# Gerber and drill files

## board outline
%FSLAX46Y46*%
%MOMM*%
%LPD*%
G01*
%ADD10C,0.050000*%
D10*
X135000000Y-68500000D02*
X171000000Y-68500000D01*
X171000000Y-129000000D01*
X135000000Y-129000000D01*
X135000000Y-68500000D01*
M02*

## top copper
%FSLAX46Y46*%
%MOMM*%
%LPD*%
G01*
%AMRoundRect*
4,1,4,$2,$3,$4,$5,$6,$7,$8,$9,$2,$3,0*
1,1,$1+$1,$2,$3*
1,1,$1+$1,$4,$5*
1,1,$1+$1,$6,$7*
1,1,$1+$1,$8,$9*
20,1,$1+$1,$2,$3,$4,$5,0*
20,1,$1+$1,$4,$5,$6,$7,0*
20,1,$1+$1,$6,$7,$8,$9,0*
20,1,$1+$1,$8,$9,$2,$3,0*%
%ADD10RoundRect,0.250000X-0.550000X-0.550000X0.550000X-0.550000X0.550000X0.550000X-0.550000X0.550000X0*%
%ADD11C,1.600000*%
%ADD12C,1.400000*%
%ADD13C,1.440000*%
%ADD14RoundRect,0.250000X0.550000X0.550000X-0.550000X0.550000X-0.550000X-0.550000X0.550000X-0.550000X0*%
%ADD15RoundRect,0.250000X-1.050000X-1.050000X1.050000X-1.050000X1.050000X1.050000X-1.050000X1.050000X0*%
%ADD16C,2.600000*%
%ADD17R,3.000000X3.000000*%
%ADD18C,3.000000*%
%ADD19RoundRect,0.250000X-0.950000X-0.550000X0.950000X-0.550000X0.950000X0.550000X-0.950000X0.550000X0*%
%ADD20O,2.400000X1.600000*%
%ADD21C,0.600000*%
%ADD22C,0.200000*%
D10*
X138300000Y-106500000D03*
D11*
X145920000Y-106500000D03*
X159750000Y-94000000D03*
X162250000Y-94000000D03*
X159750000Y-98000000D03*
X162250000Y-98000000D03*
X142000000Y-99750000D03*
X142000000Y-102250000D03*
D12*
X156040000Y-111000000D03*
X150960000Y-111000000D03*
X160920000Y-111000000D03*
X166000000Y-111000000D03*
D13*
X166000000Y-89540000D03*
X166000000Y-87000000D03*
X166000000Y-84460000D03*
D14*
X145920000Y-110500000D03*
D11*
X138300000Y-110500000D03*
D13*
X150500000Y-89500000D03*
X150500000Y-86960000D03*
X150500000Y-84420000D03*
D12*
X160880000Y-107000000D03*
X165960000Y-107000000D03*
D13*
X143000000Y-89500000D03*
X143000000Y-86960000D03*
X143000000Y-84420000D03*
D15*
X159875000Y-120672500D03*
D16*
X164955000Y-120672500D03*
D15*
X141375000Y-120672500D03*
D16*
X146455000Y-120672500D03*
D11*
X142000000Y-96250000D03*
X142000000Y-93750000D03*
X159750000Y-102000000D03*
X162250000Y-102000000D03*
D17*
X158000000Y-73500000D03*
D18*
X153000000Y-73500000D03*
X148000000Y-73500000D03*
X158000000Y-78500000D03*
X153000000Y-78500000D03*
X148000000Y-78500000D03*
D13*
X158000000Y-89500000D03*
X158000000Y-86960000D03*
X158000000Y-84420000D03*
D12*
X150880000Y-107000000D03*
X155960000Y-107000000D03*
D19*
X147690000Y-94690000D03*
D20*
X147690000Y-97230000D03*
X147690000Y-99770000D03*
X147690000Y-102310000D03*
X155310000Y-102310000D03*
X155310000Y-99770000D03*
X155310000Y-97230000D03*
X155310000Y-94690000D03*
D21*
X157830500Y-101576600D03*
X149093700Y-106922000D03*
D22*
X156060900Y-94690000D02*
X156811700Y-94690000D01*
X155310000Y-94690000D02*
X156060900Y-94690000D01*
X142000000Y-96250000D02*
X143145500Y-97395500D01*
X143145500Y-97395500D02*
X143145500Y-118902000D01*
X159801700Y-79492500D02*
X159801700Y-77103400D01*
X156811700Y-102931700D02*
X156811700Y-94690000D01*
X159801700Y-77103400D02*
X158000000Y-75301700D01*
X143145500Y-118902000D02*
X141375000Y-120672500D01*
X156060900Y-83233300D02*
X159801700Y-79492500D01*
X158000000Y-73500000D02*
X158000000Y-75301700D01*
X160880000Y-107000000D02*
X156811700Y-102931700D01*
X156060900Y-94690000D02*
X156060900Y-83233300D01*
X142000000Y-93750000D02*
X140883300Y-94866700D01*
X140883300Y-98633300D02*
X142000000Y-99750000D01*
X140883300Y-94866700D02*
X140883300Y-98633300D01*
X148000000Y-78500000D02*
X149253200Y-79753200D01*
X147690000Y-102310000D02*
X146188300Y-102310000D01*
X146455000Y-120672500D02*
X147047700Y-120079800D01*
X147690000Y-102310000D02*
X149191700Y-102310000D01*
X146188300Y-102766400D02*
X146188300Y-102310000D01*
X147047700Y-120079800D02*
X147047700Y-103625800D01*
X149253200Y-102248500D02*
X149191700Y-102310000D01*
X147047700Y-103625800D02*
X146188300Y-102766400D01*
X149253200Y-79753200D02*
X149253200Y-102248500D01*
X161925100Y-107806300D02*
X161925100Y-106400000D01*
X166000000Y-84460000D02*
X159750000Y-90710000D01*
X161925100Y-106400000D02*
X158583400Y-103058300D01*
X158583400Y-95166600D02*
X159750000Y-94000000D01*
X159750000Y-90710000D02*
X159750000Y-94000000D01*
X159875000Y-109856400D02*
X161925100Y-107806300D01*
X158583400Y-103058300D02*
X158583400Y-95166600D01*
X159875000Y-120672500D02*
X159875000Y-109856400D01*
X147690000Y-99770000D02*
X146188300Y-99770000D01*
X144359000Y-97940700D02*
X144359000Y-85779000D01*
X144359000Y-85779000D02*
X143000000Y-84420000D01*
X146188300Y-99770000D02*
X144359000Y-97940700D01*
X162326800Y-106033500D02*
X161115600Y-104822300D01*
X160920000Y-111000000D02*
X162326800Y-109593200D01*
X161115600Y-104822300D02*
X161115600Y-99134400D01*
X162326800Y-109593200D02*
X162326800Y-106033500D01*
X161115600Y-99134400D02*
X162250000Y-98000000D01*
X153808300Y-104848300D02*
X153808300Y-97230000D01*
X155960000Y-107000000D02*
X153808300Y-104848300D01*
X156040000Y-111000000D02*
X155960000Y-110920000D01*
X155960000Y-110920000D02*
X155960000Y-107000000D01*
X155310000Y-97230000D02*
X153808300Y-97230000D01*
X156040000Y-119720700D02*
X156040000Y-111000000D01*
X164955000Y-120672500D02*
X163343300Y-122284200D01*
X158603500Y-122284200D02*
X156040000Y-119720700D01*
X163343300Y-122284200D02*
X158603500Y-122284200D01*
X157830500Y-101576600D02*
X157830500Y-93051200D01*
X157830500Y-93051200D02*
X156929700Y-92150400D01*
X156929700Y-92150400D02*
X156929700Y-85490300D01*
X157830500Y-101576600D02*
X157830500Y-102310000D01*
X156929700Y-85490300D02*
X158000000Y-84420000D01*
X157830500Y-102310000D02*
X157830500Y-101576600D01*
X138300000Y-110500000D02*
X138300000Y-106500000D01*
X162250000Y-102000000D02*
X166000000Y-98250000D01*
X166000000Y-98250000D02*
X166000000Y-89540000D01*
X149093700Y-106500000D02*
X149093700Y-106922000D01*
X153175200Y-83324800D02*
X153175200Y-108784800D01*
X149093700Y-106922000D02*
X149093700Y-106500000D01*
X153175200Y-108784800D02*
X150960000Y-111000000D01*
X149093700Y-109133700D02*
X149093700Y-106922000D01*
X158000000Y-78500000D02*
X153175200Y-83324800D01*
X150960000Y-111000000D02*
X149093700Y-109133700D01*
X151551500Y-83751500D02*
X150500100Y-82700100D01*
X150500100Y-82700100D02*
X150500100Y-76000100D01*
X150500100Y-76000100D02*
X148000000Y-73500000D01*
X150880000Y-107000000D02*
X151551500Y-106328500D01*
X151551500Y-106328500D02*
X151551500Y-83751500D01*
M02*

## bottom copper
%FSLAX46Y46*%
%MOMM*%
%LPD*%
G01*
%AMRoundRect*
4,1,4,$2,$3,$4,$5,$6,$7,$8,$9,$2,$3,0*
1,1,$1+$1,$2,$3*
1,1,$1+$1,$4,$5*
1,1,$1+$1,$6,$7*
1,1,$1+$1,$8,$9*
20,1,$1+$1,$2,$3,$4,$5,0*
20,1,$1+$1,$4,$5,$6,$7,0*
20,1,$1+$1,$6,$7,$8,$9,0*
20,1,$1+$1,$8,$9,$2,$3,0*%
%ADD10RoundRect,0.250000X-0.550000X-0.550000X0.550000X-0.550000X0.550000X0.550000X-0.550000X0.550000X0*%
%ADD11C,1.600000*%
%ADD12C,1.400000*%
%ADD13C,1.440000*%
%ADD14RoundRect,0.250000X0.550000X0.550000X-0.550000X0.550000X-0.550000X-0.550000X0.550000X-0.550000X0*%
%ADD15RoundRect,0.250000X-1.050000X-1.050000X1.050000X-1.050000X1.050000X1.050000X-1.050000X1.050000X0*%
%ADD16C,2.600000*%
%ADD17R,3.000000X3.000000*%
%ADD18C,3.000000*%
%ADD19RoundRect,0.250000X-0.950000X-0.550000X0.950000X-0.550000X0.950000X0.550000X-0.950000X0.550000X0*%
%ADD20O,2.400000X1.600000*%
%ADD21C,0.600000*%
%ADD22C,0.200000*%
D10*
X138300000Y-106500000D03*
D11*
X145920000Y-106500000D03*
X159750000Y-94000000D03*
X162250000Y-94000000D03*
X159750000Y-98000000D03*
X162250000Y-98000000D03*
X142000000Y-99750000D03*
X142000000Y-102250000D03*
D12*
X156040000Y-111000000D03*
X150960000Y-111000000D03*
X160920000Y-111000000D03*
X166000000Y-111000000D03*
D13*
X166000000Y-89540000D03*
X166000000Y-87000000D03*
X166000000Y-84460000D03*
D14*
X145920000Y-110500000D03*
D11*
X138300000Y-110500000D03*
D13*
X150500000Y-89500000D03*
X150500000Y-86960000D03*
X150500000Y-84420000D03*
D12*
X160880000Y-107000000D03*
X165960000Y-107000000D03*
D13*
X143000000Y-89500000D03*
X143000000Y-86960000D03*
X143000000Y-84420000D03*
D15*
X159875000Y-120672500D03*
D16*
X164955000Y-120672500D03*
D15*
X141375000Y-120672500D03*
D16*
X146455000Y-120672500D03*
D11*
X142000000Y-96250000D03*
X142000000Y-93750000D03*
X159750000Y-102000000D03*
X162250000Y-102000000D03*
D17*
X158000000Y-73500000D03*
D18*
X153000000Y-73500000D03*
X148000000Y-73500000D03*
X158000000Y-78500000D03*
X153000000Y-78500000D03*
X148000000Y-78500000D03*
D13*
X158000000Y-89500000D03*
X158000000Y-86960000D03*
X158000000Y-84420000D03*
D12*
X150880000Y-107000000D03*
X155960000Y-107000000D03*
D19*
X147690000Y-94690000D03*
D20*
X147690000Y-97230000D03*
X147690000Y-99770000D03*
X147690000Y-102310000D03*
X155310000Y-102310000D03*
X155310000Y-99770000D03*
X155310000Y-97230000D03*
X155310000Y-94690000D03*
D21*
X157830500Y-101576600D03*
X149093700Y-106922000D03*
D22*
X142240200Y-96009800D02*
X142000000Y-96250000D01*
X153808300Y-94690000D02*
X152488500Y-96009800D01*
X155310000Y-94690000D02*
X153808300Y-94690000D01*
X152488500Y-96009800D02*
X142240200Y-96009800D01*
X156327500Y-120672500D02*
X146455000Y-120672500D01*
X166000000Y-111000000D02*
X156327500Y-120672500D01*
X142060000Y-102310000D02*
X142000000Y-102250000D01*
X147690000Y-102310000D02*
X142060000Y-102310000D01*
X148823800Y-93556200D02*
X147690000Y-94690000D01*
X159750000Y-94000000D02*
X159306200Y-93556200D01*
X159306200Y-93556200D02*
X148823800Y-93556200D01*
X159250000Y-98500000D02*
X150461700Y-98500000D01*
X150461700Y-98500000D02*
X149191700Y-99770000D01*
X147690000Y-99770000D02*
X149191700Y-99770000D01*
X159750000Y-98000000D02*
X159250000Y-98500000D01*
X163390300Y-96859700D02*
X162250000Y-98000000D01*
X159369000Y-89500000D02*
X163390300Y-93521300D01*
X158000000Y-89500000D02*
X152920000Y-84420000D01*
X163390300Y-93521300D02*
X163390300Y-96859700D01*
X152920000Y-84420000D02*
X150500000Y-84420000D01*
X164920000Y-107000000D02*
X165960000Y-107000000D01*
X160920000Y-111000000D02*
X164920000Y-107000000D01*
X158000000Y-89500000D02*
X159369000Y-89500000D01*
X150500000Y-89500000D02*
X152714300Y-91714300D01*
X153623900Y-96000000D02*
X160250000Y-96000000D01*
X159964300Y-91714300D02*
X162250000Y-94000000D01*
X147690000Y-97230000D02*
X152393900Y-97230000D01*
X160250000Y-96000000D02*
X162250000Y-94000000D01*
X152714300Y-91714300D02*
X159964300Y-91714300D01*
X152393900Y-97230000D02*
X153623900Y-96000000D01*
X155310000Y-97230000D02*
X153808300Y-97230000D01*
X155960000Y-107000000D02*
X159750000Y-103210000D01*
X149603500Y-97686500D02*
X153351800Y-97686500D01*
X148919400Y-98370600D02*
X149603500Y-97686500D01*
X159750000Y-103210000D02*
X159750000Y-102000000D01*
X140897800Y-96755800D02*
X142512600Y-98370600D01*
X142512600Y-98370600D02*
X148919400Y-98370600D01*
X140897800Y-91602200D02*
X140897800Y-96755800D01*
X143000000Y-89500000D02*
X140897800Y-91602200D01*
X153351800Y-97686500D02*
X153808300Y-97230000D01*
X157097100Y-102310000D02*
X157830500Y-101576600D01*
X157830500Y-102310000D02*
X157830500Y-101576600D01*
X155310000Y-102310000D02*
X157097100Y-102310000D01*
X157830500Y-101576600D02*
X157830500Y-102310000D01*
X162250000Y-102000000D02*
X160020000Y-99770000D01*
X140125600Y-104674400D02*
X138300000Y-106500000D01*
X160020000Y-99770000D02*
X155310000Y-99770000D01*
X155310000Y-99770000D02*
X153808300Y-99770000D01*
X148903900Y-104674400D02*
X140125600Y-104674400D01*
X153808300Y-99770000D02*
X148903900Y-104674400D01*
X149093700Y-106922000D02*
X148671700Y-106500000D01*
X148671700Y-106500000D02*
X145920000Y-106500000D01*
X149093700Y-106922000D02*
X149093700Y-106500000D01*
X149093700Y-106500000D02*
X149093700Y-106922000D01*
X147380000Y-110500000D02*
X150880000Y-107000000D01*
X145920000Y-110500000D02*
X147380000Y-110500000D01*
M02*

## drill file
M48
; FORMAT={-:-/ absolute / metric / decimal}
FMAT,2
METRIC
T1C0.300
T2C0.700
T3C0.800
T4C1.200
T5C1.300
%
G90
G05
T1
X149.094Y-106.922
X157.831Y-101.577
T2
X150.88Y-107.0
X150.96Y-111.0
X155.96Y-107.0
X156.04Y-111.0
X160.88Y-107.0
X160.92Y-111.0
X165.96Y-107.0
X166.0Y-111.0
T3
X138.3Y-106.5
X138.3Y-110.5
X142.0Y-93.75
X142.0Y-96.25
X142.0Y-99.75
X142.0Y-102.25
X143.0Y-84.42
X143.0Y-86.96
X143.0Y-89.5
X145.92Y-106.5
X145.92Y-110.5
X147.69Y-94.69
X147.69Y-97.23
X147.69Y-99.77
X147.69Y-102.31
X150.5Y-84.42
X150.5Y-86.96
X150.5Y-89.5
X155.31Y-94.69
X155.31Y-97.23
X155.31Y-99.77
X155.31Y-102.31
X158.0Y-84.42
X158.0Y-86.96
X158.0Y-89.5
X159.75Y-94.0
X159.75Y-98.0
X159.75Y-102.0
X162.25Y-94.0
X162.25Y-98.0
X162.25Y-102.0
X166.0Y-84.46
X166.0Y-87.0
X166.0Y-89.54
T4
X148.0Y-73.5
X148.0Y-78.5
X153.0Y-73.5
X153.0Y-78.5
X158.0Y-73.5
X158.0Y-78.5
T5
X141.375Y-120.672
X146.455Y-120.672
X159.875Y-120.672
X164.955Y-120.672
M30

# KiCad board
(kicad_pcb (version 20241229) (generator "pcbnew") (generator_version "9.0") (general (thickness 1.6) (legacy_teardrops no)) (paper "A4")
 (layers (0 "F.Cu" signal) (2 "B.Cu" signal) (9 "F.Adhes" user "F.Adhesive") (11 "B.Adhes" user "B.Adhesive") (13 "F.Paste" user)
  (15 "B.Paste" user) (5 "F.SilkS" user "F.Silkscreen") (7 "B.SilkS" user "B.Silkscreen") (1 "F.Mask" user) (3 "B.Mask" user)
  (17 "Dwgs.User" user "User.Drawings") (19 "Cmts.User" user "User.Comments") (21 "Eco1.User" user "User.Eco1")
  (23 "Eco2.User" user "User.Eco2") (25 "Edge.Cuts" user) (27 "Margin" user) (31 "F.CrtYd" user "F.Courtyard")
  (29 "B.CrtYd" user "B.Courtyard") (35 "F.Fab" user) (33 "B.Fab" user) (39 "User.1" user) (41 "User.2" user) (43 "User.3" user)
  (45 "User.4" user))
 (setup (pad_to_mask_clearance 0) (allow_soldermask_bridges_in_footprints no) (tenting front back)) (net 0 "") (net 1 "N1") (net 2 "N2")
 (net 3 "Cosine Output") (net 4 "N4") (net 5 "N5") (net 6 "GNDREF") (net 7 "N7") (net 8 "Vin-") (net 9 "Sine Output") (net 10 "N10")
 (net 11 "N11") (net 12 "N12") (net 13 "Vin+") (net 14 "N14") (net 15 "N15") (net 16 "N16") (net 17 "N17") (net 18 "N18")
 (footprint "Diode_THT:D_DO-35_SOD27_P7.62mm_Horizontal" (layer "F.Cu") (at 138.3 106.5)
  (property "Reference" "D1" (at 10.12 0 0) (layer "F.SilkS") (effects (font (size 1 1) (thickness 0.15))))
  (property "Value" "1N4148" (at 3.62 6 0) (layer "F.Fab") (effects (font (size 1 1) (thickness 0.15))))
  (pad "1" thru_hole roundrect (at 0 0) (size 1.6 1.6) (drill 0.8) (layers "*.Cu" "*.Mask") (remove_unused_layers no)
   (roundrect_rratio 0.15625) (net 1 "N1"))
  (pad "2" thru_hole circle (at 7.62 0) (size 1.6 1.6) (drill 0.8) (layers "*.Cu" "*.Mask") (remove_unused_layers no) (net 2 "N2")))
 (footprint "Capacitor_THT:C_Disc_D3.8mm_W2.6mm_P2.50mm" (layer "F.Cu") (at 159.75 94)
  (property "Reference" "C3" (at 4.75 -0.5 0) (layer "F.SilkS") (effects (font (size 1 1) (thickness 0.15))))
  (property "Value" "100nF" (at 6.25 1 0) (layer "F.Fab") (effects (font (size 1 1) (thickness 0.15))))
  (pad "1" thru_hole circle (at 0 0) (size 1.6 1.6) (drill 0.8) (layers "*.Cu" "*.Mask") (remove_unused_layers no) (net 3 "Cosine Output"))
  (pad "2" thru_hole circle (at 2.5 0) (size 1.6 1.6) (drill 0.8) (layers "*.Cu" "*.Mask") (remove_unused_layers no) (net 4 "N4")))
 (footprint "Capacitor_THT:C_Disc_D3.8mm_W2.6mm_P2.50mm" (layer "F.Cu") (at 159.75 98)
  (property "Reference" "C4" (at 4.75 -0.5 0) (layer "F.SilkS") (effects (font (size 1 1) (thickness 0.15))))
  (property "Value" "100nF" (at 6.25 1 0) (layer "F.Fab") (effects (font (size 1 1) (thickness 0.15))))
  (pad "1" thru_hole circle (at 0 0) (size 1.6 1.6) (drill 0.8) (layers "*.Cu" "*.Mask") (remove_unused_layers no) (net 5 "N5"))
  (pad "2" thru_hole circle (at 2.5 0) (size 1.6 1.6) (drill 0.8) (layers "*.Cu" "*.Mask") (remove_unused_layers no) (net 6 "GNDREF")))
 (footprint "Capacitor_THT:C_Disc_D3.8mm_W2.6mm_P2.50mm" (layer "F.Cu") (at 142 99.75 -90)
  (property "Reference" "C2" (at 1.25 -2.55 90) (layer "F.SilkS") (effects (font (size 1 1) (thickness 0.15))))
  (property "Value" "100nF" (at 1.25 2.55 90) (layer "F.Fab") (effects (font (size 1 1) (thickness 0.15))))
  (pad "1" thru_hole circle (at 0 0 270) (size 1.6 1.6) (drill 0.8) (layers "*.Cu" "*.Mask") (remove_unused_layers no) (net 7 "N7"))
  (pad "2" thru_hole circle (at 2.5 0 270) (size 1.6 1.6) (drill 0.8) (layers "*.Cu" "*.Mask") (remove_unused_layers no) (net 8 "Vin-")))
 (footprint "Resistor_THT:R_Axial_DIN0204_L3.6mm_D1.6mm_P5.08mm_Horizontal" (layer "F.Cu") (at 156.04 111 180)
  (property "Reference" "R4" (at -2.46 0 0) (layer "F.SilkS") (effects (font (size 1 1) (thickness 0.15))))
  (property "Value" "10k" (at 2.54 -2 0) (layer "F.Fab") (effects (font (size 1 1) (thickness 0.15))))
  (pad "1" thru_hole circle (at 0 0 180) (size 1.4 1.4) (drill 0.7) (layers "*.Cu" "*.Mask") (remove_unused_layers no) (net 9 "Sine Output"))
  (pad "2" thru_hole circle (at 5.08 0 180) (size 1.4 1.4) (drill 0.7) (layers "*.Cu" "*.Mask") (remove_unused_layers no) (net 2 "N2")))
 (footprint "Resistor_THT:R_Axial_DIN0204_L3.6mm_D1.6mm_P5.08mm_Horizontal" (layer "F.Cu") (at 160.92 111)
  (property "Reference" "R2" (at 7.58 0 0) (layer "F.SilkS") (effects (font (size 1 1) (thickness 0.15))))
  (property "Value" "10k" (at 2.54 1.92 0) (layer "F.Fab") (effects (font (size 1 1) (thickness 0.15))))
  (pad "1" thru_hole circle (at 0 0) (size 1.4 1.4) (drill 0.7) (layers "*.Cu" "*.Mask") (remove_unused_layers no) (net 6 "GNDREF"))
  (pad "2" thru_hole circle (at 5.08 0) (size 1.4 1.4) (drill 0.7) (layers "*.Cu" "*.Mask") (remove_unused_layers no) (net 8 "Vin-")))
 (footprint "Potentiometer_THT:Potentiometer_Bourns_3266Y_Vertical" (layer "F.Cu") (at 166 89.54 -90)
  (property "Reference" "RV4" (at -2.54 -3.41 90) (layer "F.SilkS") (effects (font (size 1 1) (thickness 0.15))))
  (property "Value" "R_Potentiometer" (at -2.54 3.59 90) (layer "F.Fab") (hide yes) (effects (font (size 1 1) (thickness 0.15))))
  (pad "1" thru_hole circle (at 0 0 270) (size 1.44 1.44) (drill 0.8) (layers "*.Cu" "*.Mask") (remove_unused_layers no) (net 1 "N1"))
  (pad "2" thru_hole circle (at -2.54 0 270) (size 1.44 1.44) (drill 0.8) (layers "*.Cu" "*.Mask") (remove_unused_layers no) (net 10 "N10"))
  (pad "3" thru_hole circle (at -5.08 0 270) (size 1.44 1.44) (drill 0.8) (layers "*.Cu" "*.Mask") (remove_unused_layers no)
   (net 3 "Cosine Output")))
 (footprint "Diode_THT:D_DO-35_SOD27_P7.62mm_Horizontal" (layer "F.Cu") (at 145.92 110.5 180)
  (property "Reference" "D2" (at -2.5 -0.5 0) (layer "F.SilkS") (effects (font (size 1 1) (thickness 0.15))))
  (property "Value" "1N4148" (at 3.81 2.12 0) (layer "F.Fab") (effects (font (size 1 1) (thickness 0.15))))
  (pad "1" thru_hole roundrect (at 0 0 180) (size 1.6 1.6) (drill 0.8) (layers "*.Cu" "*.Mask") (remove_unused_layers no)
   (roundrect_rratio 0.15625) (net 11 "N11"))
  (pad "2" thru_hole circle (at 7.62 0 180) (size 1.6 1.6) (drill 0.8) (layers "*.Cu" "*.Mask") (remove_unused_layers no) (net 1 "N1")))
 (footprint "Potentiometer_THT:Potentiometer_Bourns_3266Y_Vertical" (layer "F.Cu") (at 150.5 89.5 -90)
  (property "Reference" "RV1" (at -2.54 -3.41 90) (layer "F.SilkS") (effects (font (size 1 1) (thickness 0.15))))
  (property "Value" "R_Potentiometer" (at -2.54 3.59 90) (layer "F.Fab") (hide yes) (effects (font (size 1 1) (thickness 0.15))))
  (pad "1" thru_hole circle (at 0 0 270) (size 1.44 1.44) (drill 0.8) (layers "*.Cu" "*.Mask") (remove_unused_layers no) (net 4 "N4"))
  (pad "2" thru_hole circle (at -2.54 0 270) (size 1.44 1.44) (drill 0.8) (layers "*.Cu" "*.Mask") (remove_unused_layers no) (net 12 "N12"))
  (pad "3" thru_hole circle (at -5.08 0 270) (size 1.44 1.44) (drill 0.8) (layers "*.Cu" "*.Mask") (remove_unused_layers no)
   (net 6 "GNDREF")))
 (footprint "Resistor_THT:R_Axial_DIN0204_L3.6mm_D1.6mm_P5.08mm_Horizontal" (layer "F.Cu") (at 160.88 107)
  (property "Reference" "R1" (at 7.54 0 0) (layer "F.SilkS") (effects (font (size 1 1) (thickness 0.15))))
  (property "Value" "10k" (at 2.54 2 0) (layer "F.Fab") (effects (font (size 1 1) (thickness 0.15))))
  (pad "1" thru_hole circle (at 0 0) (size 1.4 1.4) (drill 0.7) (layers "*.Cu" "*.Mask") (remove_unused_layers no) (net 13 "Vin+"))
  (pad "2" thru_hole circle (at 5.08 0) (size 1.4 1.4) (drill 0.7) (layers "*.Cu" "*.Mask") (remove_unused_layers no) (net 6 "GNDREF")))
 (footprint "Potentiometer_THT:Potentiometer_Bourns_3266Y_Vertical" (layer "F.Cu") (at 143 89.5 -90)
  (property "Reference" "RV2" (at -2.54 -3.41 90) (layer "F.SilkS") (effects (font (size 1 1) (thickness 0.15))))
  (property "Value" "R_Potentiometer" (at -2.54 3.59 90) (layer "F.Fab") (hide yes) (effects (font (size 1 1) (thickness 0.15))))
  (pad "1" thru_hole circle (at 0 0 270) (size 1.44 1.44) (drill 0.8) (layers "*.Cu" "*.Mask") (remove_unused_layers no)
   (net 9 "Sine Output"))
  (pad "2" thru_hole circle (at -2.54 0 270) (size 1.44 1.44) (drill 0.8) (layers "*.Cu" "*.Mask") (remove_unused_layers no) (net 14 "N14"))
  (pad "3" thru_hole circle (at -5.08 0 270) (size 1.44 1.44) (drill 0.8) (layers "*.Cu" "*.Mask") (remove_unused_layers no) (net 5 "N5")))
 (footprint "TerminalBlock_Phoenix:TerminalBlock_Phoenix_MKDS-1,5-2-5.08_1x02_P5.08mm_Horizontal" (layer "F.Cu") (at 159.875 120.6725)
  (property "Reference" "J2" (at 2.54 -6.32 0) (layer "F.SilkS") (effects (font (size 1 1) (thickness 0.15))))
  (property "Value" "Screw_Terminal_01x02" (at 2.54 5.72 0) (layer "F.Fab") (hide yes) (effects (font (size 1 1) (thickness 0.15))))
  (pad "1" thru_hole roundrect (at 0 0) (size 2.6 2.6) (drill 1.3) (layers "*.Cu" "*.Mask") (remove_unused_layers no)
   (roundrect_rratio 0.096154) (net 3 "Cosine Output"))
  (pad "2" thru_hole circle (at 5.08 0) (size 2.6 2.6) (drill 1.3) (layers "*.Cu" "*.Mask") (remove_unused_layers no) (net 9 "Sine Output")))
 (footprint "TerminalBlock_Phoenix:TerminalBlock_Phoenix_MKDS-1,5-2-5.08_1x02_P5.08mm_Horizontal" (layer "F.Cu") (at 141.375 120.6725)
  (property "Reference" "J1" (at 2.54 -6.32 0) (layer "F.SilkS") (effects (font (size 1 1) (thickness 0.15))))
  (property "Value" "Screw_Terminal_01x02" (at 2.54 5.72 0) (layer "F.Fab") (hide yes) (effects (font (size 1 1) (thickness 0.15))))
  (pad "1" thru_hole roundrect (at 0 0) (size 2.6 2.6) (drill 1.3) (layers "*.Cu" "*.Mask") (remove_unused_layers no)
   (roundrect_rratio 0.096154) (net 13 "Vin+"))
  (pad "2" thru_hole circle (at 5.08 0) (size 2.6 2.6) (drill 1.3) (layers "*.Cu" "*.Mask") (remove_unused_layers no) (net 8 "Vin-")))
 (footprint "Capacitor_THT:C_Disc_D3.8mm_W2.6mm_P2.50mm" (layer "F.Cu") (at 142 96.25 90)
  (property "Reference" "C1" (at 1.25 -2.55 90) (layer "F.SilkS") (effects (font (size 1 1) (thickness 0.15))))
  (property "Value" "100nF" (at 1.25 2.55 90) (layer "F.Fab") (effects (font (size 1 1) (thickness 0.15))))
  (pad "1" thru_hole circle (at 0 0 90) (size 1.6 1.6) (drill 0.8) (layers "*.Cu" "*.Mask") (remove_unused_layers no) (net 13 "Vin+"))
  (pad "2" thru_hole circle (at 2.5 0 90) (size 1.6 1.6) (drill 0.8) (layers "*.Cu" "*.Mask") (remove_unused_layers no) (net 7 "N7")))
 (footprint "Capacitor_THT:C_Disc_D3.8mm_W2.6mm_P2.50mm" (layer "F.Cu") (at 159.75 102)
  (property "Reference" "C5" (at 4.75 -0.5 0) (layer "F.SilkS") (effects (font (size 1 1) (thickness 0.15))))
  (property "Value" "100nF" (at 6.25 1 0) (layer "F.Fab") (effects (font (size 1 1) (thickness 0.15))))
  (pad "1" thru_hole circle (at 0 0) (size 1.6 1.6) (drill 0.8) (layers "*.Cu" "*.Mask") (remove_unused_layers no) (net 9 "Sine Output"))
  (pad "2" thru_hole circle (at 2.5 0) (size 1.6 1.6) (drill 0.8) (layers "*.Cu" "*.Mask") (remove_unused_layers no) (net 1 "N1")))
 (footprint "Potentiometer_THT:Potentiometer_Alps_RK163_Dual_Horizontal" (layer "F.Cu") (at 158 73.5 -90)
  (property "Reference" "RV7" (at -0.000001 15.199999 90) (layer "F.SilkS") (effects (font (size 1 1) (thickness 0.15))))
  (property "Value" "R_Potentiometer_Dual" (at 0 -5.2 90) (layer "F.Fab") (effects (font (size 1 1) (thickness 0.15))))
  (pad "1" thru_hole rect (at 0 0 90) (size 3 3) (drill 1.2) (layers "*.Cu" "*.Mask") (remove_unused_layers no) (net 13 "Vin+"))
  (pad "2" thru_hole circle (at 0 5 90) (size 3 3) (drill 1.2) (layers "*.Cu" "*.Mask") (remove_unused_layers no) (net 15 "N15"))
  (pad "3" thru_hole circle (at 0 10 90) (size 3 3) (drill 1.2) (layers "*.Cu" "*.Mask") (remove_unused_layers no) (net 11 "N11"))
  (pad "4" thru_hole circle (at 5 0 90) (size 3 3) (drill 1.2) (layers "*.Cu" "*.Mask") (remove_unused_layers no) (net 2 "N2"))
  (pad "5" thru_hole circle (at 5 5 90) (size 3 3) (drill 1.2) (layers "*.Cu" "*.Mask") (remove_unused_layers no) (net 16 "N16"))
  (pad "6" thru_hole circle (at 5 10 90) (size 3 3) (drill 1.2) (layers "*.Cu" "*.Mask") (remove_unused_layers no) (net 8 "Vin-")))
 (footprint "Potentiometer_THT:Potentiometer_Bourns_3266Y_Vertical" (layer "F.Cu") (at 158 89.5 -90)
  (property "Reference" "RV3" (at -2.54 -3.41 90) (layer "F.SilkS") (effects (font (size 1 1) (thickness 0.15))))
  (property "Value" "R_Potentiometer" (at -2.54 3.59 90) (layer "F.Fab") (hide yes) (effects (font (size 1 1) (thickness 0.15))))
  (pad "1" thru_hole circle (at 0 0 270) (size 1.44 1.44) (drill 0.8) (layers "*.Cu" "*.Mask") (remove_unused_layers no) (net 6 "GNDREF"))
  (pad "2" thru_hole circle (at -2.54 0 270) (size 1.44 1.44) (drill 0.8) (layers "*.Cu" "*.Mask") (remove_unused_layers no) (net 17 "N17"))
  (pad "3" thru_hole circle (at -5.08 0 270) (size 1.44 1.44) (drill 0.8) (layers "*.Cu" "*.Mask") (remove_unused_layers no) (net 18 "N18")))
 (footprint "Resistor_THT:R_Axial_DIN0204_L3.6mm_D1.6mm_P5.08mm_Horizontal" (layer "F.Cu") (at 150.88 107)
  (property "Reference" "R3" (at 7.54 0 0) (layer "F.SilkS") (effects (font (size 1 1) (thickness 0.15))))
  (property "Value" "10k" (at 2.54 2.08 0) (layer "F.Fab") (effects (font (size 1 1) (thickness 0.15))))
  (pad "1" thru_hole circle (at 0 0) (size 1.4 1.4) (drill 0.7) (layers "*.Cu" "*.Mask") (remove_unused_layers no) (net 11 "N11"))
  (pad "2" thru_hole circle (at 5.08 0) (size 1.4 1.4) (drill 0.7) (layers "*.Cu" "*.Mask") (remove_unused_layers no) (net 9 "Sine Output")))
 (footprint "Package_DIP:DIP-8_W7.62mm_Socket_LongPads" (layer "F.Cu") (at 147.69 94.69)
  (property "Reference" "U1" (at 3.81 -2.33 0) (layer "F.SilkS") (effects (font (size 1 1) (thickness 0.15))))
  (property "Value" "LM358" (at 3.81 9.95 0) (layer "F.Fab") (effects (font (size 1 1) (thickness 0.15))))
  (pad "1" thru_hole roundrect (at 0 0) (size 2.4 1.6) (drill 0.8) (layers "*.Cu" "*.Mask") (remove_unused_layers no)
   (roundrect_rratio 0.15625) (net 3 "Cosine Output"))
  (pad "2" thru_hole oval (at 0 2.54) (size 2.4 1.6) (drill 0.8) (layers "*.Cu" "*.Mask") (remove_unused_layers no) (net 4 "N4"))
  (pad "3" thru_hole oval (at 0 5.08) (size 2.4 1.6) (drill 0.8) (layers "*.Cu" "*.Mask") (remove_unused_layers no) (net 5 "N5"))
  (pad "4" thru_hole oval (at 0 7.62) (size 2.4 1.6) (drill 0.8) (layers "*.Cu" "*.Mask") (remove_unused_layers no) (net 8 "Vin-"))
  (pad "5" thru_hole oval (at 7.62 7.62) (size 2.4 1.6) (drill 0.8) (layers "*.Cu" "*.Mask") (remove_unused_layers no) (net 18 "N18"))
  (pad "6" thru_hole oval (at 7.62 5.08) (size 2.4 1.6) (drill 0.8) (layers "*.Cu" "*.Mask") (remove_unused_layers no) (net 1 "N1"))
  (pad "7" thru_hole oval (at 7.62 2.54) (size 2.4 1.6) (drill 0.8) (layers "*.Cu" "*.Mask") (remove_unused_layers no) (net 9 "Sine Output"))
  (pad "8" thru_hole oval (at 7.62 0) (size 2.4 1.6) (drill 0.8) (layers "*.Cu" "*.Mask") (remove_unused_layers no) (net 13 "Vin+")))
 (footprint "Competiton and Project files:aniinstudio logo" (layer "B.Cu") (at 167.5 72 -90)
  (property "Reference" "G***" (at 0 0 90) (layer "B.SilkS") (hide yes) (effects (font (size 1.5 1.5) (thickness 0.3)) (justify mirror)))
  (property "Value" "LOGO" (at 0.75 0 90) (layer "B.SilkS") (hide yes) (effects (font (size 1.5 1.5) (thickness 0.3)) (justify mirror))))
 (gr_rect (start 135 68.5) (end 171 129) (stroke (width 0.05) (type default)) (fill no) (layer "Edge.Cuts"))
 (segment (start 156.0609 94.69) (end 156.8117 94.69) (width 0.2) (layer "F.Cu") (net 13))
 (segment (start 155.31 94.69) (end 156.0609 94.69) (width 0.2) (layer "F.Cu") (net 13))
 (segment (start 142 96.25) (end 143.1455 97.3955) (width 0.2) (layer "F.Cu") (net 13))
 (segment (start 143.1455 97.3955) (end 143.1455 118.902) (width 0.2) (layer "F.Cu") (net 13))
 (segment (start 159.8017 79.4925) (end 159.8017 77.1034) (width 0.2) (layer "F.Cu") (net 13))
 (segment (start 156.8117 102.9317) (end 156.8117 94.69) (width 0.2) (layer "F.Cu") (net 13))
 (segment (start 159.8017 77.1034) (end 158 75.3017) (width 0.2) (layer "F.Cu") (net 13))
 (segment (start 143.1455 118.902) (end 141.375 120.6725) (width 0.2) (layer "F.Cu") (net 13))
 (segment (start 156.0609 83.2333) (end 159.8017 79.4925) (width 0.2) (layer "F.Cu") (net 13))
 (segment (start 158 73.5) (end 158 75.3017) (width 0.2) (layer "F.Cu") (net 13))
 (segment (start 160.88 107) (end 156.8117 102.9317) (width 0.2) (layer "F.Cu") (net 13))
 (segment (start 156.0609 94.69) (end 156.0609 83.2333) (width 0.2) (layer "F.Cu") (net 13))
 (segment (start 142.2402 96.0098) (end 142 96.25) (width 0.2) (layer "B.Cu") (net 13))
 (segment (start 153.8083 94.69) (end 152.4885 96.0098) (width 0.2) (layer "B.Cu") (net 13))
 (segment (start 155.31 94.69) (end 153.8083 94.69) (width 0.2) (layer "B.Cu") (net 13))
 (segment (start 152.4885 96.0098) (end 142.2402 96.0098) (width 0.2) (layer "B.Cu") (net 13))
 (segment (start 142 93.75) (end 140.8833 94.8667) (width 0.2) (layer "F.Cu") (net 7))
 (segment (start 140.8833 98.6333) (end 142 99.75) (width 0.2) (layer "F.Cu") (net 7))
 (segment (start 140.8833 94.8667) (end 140.8833 98.6333) (width 0.2) (layer "F.Cu") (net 7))
 (segment (start 148 78.5) (end 149.2532 79.7532) (width 0.2) (layer "F.Cu") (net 8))
 (segment (start 147.69 102.31) (end 146.1883 102.31) (width 0.2) (layer "F.Cu") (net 8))
 (segment (start 146.455 120.6725) (end 147.0477 120.0798) (width 0.2) (layer "F.Cu") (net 8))
 (segment (start 147.69 102.31) (end 149.1917 102.31) (width 0.2) (layer "F.Cu") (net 8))
 (segment (start 146.1883 102.7664) (end 146.1883 102.31) (width 0.2) (layer "F.Cu") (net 8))
 (segment (start 147.0477 120.0798) (end 147.0477 103.6258) (width 0.2) (layer "F.Cu") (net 8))
 (segment (start 149.2532 102.2485) (end 149.1917 102.31) (width 0.2) (layer "F.Cu") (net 8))
 (segment (start 147.0477 103.6258) (end 146.1883 102.7664) (width 0.2) (layer "F.Cu") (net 8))
 (segment (start 149.2532 79.7532) (end 149.2532 102.2485) (width 0.2) (layer "F.Cu") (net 8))
 (segment (start 156.3275 120.6725) (end 146.455 120.6725) (width 0.2) (layer "B.Cu") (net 8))
 (segment (start 166 111) (end 156.3275 120.6725) (width 0.2) (layer "B.Cu") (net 8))
 (segment (start 142.06 102.31) (end 142 102.25) (width 0.2) (layer "B.Cu") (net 8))
 (segment (start 147.69 102.31) (end 142.06 102.31) (width 0.2) (layer "B.Cu") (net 8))
 (segment (start 161.9251 107.8063) (end 161.9251 106.4) (width 0.2) (layer "F.Cu") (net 3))
 (segment (start 166 84.46) (end 159.75 90.71) (width 0.2) (layer "F.Cu") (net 3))
 (segment (start 161.9251 106.4) (end 158.5834 103.0583) (width 0.2) (layer "F.Cu") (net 3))
 (segment (start 158.5834 95.1666) (end 159.75 94) (width 0.2) (layer "F.Cu") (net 3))
 (segment (start 159.75 90.71) (end 159.75 94) (width 0.2) (layer "F.Cu") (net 3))
 (segment (start 159.875 109.8564) (end 161.9251 107.8063) (width 0.2) (layer "F.Cu") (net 3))
 (segment (start 158.5834 103.0583) (end 158.5834 95.1666) (width 0.2) (layer "F.Cu") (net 3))
 (segment (start 159.875 120.6725) (end 159.875 109.8564) (width 0.2) (layer "F.Cu") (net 3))
 (segment (start 148.8238 93.5562) (end 147.69 94.69) (width 0.2) (layer "B.Cu") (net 3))
 (segment (start 159.75 94) (end 159.3062 93.5562) (width 0.2) (layer "B.Cu") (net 3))
 (segment (start 159.3062 93.5562) (end 148.8238 93.5562) (width 0.2) (layer "B.Cu") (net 3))
 (segment (start 147.69 99.77) (end 146.1883 99.77) (width 0.2) (layer "F.Cu") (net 5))
 (segment (start 144.359 97.9407) (end 144.359 85.779) (width 0.2) (layer "F.Cu") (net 5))
 (segment (start 144.359 85.779) (end 143 84.42) (width 0.2) (layer "F.Cu") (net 5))
 (segment (start 146.1883 99.77) (end 144.359 97.9407) (width 0.2) (layer "F.Cu") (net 5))
 (segment (start 159.25 98.5) (end 150.4617 98.5) (width 0.2) (layer "B.Cu") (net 5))
 (segment (start 150.4617 98.5) (end 149.1917 99.77) (width 0.2) (layer "B.Cu") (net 5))
 (segment (start 147.69 99.77) (end 149.1917 99.77) (width 0.2) (layer "B.Cu") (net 5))
 (segment (start 159.75 98) (end 159.25 98.5) (width 0.2) (layer "B.Cu") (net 5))
 (segment (start 162.3268 106.0335) (end 161.1156 104.8223) (width 0.2) (layer "F.Cu") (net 6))
 (segment (start 160.92 111) (end 162.3268 109.5932) (width 0.2) (layer "F.Cu") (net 6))
 (segment (start 161.1156 104.8223) (end 161.1156 99.1344) (width 0.2) (layer "F.Cu") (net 6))
 (segment (start 162.3268 109.5932) (end 162.3268 106.0335) (width 0.2) (layer "F.Cu") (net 6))
 (segment (start 161.1156 99.1344) (end 162.25 98) (width 0.2) (layer "F.Cu") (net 6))
 (segment (start 163.3903 96.8597) (end 162.25 98) (width 0.2) (layer "B.Cu") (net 6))
 (segment (start 159.369 89.5) (end 163.3903 93.5213) (width 0.2) (layer "B.Cu") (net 6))
 (segment (start 158 89.5) (end 152.92 84.42) (width 0.2) (layer "B.Cu") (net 6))
 (segment (start 163.3903 93.5213) (end 163.3903 96.8597) (width 0.2) (layer "B.Cu") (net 6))
 (segment (start 152.92 84.42) (end 150.5 84.42) (width 0.2) (layer "B.Cu") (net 6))
 (segment (start 164.92 107) (end 165.96 107) (width 0.2) (layer "B.Cu") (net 6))
 (segment (start 160.92 111) (end 164.92 107) (width 0.2) (layer "B.Cu") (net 6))
 (segment (start 158 89.5) (end 159.369 89.5) (width 0.2) (layer "B.Cu") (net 6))
 (segment (start 150.5 89.5) (end 152.7143 91.7143) (width 0.2) (layer "B.Cu") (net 4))
 (segment (start 153.6239 96) (end 160.25 96) (width 0.2) (layer "B.Cu") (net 4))
 (segment (start 159.9643 91.7143) (end 162.25 94) (width 0.2) (layer "B.Cu") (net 4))
 (segment (start 147.69 97.23) (end 152.3939 97.23) (width 0.2) (layer "B.Cu") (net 4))
 (segment (start 160.25 96) (end 162.25 94) (width 0.2) (layer "B.Cu") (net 4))
 (segment (start 152.7143 91.7143) (end 159.9643 91.7143) (width 0.2) (layer "B.Cu") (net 4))
 (segment (start 152.3939 97.23) (end 153.6239 96) (width 0.2) (layer "B.Cu") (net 4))
 (segment (start 153.8083 104.8483) (end 153.8083 97.23) (width 0.2) (layer "F.Cu") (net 9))
 (segment (start 155.96 107) (end 153.8083 104.8483) (width 0.2) (layer "F.Cu") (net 9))
 (segment (start 156.04 111) (end 155.96 110.92) (width 0.2) (layer "F.Cu") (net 9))
 (segment (start 155.96 110.92) (end 155.96 107) (width 0.2) (layer "F.Cu") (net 9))
 (segment (start 155.31 97.23) (end 153.8083 97.23) (width 0.2) (layer "F.Cu") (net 9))
 (segment (start 156.04 119.7207) (end 156.04 111) (width 0.2) (layer "F.Cu") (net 9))
 (segment (start 164.955 120.6725) (end 163.3433 122.2842) (width 0.2) (layer "F.Cu") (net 9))
 (segment (start 158.6035 122.2842) (end 156.04 119.7207) (width 0.2) (layer "F.Cu") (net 9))
 (segment (start 163.3433 122.2842) (end 158.6035 122.2842) (width 0.2) (layer "F.Cu") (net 9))
 (segment (start 155.31 97.23) (end 153.8083 97.23) (width 0.2) (layer "B.Cu") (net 9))
 (segment (start 155.96 107) (end 159.75 103.21) (width 0.2) (layer "B.Cu") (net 9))
 (segment (start 149.6035 97.6865) (end 153.3518 97.6865) (width 0.2) (layer "B.Cu") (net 9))
 (segment (start 148.9194 98.3706) (end 149.6035 97.6865) (width 0.2) (layer "B.Cu") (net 9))
 (segment (start 159.75 103.21) (end 159.75 102) (width 0.2) (layer "B.Cu") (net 9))
 (segment (start 140.8978 96.7558) (end 142.5126 98.3706) (width 0.2) (layer "B.Cu") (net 9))
 (segment (start 142.5126 98.3706) (end 148.9194 98.3706) (width 0.2) (layer "B.Cu") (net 9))
 (segment (start 140.8978 91.6022) (end 140.8978 96.7558) (width 0.2) (layer "B.Cu") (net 9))
 (segment (start 143 89.5) (end 140.8978 91.6022) (width 0.2) (layer "B.Cu") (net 9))
 (segment (start 153.3518 97.6865) (end 153.8083 97.23) (width 0.2) (layer "B.Cu") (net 9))
 (segment (start 157.8305 101.5766) (end 157.8305 93.0512) (width 0.2) (layer "F.Cu") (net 18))
 (segment (start 157.8305 93.0512) (end 156.9297 92.1504) (width 0.2) (layer "F.Cu") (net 18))
 (segment (start 156.9297 92.1504) (end 156.9297 85.4903) (width 0.2) (layer "F.Cu") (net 18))
 (segment (start 157.8305 101.5766) (end 157.8305 102.31) (width 0.2) (layer "F.Cu") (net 18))
 (segment (start 156.9297 85.4903) (end 158 84.42) (width 0.2) (layer "F.Cu") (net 18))
 (segment (start 157.8305 102.31) (end 157.8305 101.5766) (width 0.2) (layer "F.Cu") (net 18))
 (via (at 157.8305 101.5766) (size 0.6) (drill 0.3) (layers "F.Cu" "B.Cu") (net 18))
 (segment (start 157.0971 102.31) (end 157.8305 101.5766) (width 0.2) (layer "B.Cu") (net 18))
 (segment (start 157.8305 102.31) (end 157.8305 101.5766) (width 0.2) (layer "B.Cu") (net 18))
 (segment (start 155.31 102.31) (end 157.0971 102.31) (width 0.2) (layer "B.Cu") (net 18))
 (segment (start 157.8305 101.5766) (end 157.8305 102.31) (width 0.2) (layer "B.Cu") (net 18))
 (segment (start 138.3 110.5) (end 138.3 106.5) (width 0.2) (layer "F.Cu") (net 1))
 (segment (start 162.25 102) (end 166 98.25) (width 0.2) (layer "F.Cu") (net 1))
 (segment (start 166 98.25) (end 166 89.54) (width 0.2) (layer "F.Cu") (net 1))
 (segment (start 162.25 102) (end 160.02 99.77) (width 0.2) (layer "B.Cu") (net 1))
 (segment (start 140.1256 104.6744) (end 138.3 106.5) (width 0.2) (layer "B.Cu") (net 1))
 (segment (start 160.02 99.77) (end 155.31 99.77) (width 0.2) (layer "B.Cu") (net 1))
 (segment (start 155.31 99.77) (end 153.8083 99.77) (width 0.2) (layer "B.Cu") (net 1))
 (segment (start 148.9039 104.6744) (end 140.1256 104.6744) (width 0.2) (layer "B.Cu") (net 1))
 (segment (start 153.8083 99.77) (end 148.9039 104.6744) (width 0.2) (layer "B.Cu") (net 1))
 (segment (start 149.0937 106.5) (end 149.0937 106.922) (width 0.2) (layer "F.Cu") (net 2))
 (segment (start 153.1752 83.3248) (end 153.1752 108.7848) (width 0.2) (layer "F.Cu") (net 2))
 (segment (start 149.0937 106.922) (end 149.0937 106.5) (width 0.2) (layer "F.Cu") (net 2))
 (segment (start 153.1752 108.7848) (end 150.96 111) (width 0.2) (layer "F.Cu") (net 2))
 (segment (start 149.0937 109.1337) (end 149.0937 106.922) (width 0.2) (layer "F.Cu") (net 2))
 (segment (start 158 78.5) (end 153.1752 83.3248) (width 0.2) (layer "F.Cu") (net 2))
 (segment (start 150.96 111) (end 149.0937 109.1337) (width 0.2) (layer "F.Cu") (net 2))
 (via (at 149.0937 106.922) (size 0.6) (drill 0.3) (layers "F.Cu" "B.Cu") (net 2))
 (segment (start 149.0937 106.922) (end 148.6717 106.5) (width 0.2) (layer "B.Cu") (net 2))
 (segment (start 148.6717 106.5) (end 145.92 106.5) (width 0.2) (layer "B.Cu") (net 2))
 (segment (start 149.0937 106.922) (end 149.0937 106.5) (width 0.2) (layer "B.Cu") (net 2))
 (segment (start 149.0937 106.5) (end 149.0937 106.922) (width 0.2) (layer "B.Cu") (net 2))
 (segment (start 151.5515 83.7515) (end 150.5001 82.7001) (width 0.2) (layer "F.Cu") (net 11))
 (segment (start 150.5001 82.7001) (end 150.5001 76.0001) (width 0.2) (layer "F.Cu") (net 11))
 (segment (start 150.5001 76.0001) (end 148 73.5) (width 0.2) (layer "F.Cu") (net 11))
 (segment (start 150.88 107) (end 151.5515 106.3285) (width 0.2) (layer "F.Cu") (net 11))
 (segment (start 151.5515 106.3285) (end 151.5515 83.7515) (width 0.2) (layer "F.Cu") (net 11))
 (segment (start 147.38 110.5) (end 150.88 107) (width 0.2) (layer "B.Cu") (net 11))
 (segment (start 145.92 110.5) (end 147.38 110.5) (width 0.2) (layer "B.Cu") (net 11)))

